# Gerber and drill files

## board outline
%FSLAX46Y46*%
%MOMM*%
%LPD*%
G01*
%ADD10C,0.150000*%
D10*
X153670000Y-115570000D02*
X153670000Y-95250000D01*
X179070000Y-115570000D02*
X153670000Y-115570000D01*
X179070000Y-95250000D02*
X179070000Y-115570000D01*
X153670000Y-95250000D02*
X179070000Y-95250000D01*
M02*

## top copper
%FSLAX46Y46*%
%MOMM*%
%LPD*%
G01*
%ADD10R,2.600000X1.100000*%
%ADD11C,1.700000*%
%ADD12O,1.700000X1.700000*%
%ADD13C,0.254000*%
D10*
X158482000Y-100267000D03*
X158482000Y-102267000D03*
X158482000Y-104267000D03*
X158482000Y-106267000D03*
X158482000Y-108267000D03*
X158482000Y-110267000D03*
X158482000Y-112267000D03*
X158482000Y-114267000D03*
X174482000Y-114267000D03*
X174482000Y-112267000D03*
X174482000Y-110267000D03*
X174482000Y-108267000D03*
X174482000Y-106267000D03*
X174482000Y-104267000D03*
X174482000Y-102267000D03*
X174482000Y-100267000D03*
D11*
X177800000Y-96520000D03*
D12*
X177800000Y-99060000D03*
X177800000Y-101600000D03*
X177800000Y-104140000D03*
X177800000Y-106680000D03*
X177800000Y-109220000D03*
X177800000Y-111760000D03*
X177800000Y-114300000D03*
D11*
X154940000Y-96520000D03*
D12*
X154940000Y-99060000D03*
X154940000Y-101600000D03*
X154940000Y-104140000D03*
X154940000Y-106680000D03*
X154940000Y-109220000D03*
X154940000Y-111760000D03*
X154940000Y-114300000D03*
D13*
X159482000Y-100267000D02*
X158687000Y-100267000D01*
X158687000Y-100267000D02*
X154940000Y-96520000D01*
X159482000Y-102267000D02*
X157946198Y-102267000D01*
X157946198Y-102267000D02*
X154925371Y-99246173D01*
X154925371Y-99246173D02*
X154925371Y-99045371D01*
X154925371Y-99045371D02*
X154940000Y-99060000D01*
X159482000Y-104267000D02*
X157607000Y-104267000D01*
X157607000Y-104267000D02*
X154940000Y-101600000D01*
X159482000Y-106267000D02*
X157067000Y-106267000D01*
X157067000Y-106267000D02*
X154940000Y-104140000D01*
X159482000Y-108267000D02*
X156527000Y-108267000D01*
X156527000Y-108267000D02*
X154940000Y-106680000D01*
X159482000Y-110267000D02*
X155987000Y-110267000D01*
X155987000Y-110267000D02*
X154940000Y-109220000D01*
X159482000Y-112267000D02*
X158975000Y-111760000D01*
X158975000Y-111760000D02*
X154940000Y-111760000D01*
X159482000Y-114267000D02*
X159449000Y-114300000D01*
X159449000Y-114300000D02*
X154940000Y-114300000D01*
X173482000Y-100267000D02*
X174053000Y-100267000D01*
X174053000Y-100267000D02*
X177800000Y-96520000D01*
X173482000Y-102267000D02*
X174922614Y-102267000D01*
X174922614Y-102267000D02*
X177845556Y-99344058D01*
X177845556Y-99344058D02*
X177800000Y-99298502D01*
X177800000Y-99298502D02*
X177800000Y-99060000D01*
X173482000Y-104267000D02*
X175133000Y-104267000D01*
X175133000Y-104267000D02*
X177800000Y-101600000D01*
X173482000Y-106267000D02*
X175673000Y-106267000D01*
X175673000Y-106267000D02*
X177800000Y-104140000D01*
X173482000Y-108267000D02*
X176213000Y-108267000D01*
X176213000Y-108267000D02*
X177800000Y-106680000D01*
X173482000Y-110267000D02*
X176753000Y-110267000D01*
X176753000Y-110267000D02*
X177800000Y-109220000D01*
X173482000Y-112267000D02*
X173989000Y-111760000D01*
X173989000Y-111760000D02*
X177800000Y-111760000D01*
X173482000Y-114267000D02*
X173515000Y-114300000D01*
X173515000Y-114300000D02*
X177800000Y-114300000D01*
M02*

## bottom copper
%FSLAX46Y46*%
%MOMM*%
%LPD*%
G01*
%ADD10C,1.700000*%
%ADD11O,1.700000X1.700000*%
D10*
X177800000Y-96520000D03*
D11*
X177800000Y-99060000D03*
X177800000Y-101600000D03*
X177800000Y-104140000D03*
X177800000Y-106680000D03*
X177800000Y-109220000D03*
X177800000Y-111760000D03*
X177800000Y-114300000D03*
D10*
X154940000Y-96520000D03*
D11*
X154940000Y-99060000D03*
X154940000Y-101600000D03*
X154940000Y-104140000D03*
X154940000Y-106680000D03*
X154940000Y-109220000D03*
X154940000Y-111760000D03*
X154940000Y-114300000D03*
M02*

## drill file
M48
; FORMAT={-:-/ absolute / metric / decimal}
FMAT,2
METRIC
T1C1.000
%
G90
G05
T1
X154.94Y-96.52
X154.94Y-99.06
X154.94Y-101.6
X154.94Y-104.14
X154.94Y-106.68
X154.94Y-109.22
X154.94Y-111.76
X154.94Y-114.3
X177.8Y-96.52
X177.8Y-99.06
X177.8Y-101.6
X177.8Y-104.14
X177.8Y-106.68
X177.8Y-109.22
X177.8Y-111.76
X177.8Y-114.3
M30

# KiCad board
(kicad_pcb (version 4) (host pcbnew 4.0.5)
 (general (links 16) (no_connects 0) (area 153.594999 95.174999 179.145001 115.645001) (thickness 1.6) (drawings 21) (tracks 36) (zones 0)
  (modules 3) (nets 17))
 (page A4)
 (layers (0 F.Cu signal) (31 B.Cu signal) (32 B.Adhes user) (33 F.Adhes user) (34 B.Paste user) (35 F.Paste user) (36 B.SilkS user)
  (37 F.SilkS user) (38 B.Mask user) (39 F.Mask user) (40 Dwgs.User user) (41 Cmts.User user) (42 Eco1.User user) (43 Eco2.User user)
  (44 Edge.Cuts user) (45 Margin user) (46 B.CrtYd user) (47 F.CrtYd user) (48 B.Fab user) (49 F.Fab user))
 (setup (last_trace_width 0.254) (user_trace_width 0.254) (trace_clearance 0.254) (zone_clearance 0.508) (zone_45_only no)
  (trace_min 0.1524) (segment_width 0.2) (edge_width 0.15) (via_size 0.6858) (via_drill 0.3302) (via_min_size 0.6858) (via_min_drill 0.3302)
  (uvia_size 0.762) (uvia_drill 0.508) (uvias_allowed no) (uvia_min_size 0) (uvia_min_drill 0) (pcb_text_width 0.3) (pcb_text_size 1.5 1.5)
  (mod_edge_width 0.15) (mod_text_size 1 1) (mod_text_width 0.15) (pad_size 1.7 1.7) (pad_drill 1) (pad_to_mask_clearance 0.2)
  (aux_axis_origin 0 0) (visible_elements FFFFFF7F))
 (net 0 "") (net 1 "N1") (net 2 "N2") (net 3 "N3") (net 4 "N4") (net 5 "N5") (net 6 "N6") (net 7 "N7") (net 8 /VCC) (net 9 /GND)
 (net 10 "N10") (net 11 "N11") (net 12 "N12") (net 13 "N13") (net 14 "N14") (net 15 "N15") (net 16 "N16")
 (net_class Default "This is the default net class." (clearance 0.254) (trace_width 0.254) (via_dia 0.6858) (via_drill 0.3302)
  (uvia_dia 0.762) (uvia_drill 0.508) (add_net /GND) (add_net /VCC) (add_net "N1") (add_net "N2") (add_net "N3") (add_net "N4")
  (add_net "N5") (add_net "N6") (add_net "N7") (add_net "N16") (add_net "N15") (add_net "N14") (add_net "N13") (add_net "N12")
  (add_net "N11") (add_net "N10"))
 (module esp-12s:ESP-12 (layer F.Cu) (at 159.482 100.267)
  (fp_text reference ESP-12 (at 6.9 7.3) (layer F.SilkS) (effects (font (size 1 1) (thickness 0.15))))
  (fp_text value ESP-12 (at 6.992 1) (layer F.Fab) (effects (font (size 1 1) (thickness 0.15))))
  (pad 1 smd rect (at 0 0) (size 2.6 1.1) (drill (offset -1 0)) (layers F.Cu F.Paste F.Mask) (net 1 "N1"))
  (pad 2 smd rect (at 0 2) (size 2.6 1.1) (drill (offset -1 0)) (layers F.Cu F.Paste F.Mask) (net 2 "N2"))
  (pad 3 smd rect (at 0 4) (size 2.6 1.1) (drill (offset -1 0)) (layers F.Cu F.Paste F.Mask) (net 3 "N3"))
  (pad 4 smd rect (at 0 6) (size 2.6 1.1) (drill (offset -1 0)) (layers F.Cu F.Paste F.Mask) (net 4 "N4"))
  (pad 5 smd rect (at 0 8) (size 2.6 1.1) (drill (offset -1 0)) (layers F.Cu F.Paste F.Mask) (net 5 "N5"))
  (pad 6 smd rect (at 0 10) (size 2.6 1.1) (drill (offset -1 0)) (layers F.Cu F.Paste F.Mask) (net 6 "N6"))
  (pad 7 smd rect (at 0 12) (size 2.6 1.1) (drill (offset -1 0)) (layers F.Cu F.Paste F.Mask) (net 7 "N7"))
  (pad 8 smd rect (at 0 14) (size 2.6 1.1) (drill (offset -1 0)) (layers F.Cu F.Paste F.Mask) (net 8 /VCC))
  (pad 9 smd rect (at 14 14) (size 2.6 1.1) (drill (offset 1 0)) (layers F.Cu F.Paste F.Mask) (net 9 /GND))
  (pad 10 smd rect (at 14 12) (size 2.6 1.1) (drill (offset 1 0)) (layers F.Cu F.Paste F.Mask) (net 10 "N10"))
  (pad 11 smd rect (at 14 10) (size 2.6 1.1) (drill (offset 1 0)) (layers F.Cu F.Paste F.Mask) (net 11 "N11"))
  (pad 12 smd rect (at 14 8) (size 2.6 1.1) (drill (offset 1 0)) (layers F.Cu F.Paste F.Mask) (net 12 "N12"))
  (pad 13 smd rect (at 14 6) (size 2.6 1.1) (drill (offset 1 0)) (layers F.Cu F.Paste F.Mask) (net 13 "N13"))
  (pad 14 smd rect (at 14 4) (size 2.6 1.1) (drill (offset 1 0)) (layers F.Cu F.Paste F.Mask) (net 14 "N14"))
  (pad 15 smd rect (at 14 2) (size 2.6 1.1) (drill (offset 1 0)) (layers F.Cu F.Paste F.Mask) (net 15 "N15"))
  (pad 16 smd rect (at 14 0) (size 2.6 1.1) (drill (offset 1 0)) (layers F.Cu F.Paste F.Mask) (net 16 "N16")))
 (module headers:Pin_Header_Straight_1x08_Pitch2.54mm (layer F.Cu) (at 177.8 96.52)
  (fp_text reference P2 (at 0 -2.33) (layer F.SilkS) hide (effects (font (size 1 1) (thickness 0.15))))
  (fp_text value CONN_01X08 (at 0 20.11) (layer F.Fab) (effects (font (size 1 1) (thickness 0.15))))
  (pad 1 thru_hole circle (at 0 0) (size 1.7 1.7) (drill 1) (layers *.Cu *.Mask) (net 16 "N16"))
  (pad 2 thru_hole oval (at 0 2.54) (size 1.7 1.7) (drill 1) (layers *.Cu *.Mask) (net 15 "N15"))
  (pad 3 thru_hole oval (at 0 5.08) (size 1.7 1.7) (drill 1) (layers *.Cu *.Mask) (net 14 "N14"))
  (pad 4 thru_hole oval (at 0 7.62) (size 1.7 1.7) (drill 1) (layers *.Cu *.Mask) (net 13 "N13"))
  (pad 5 thru_hole oval (at 0 10.16) (size 1.7 1.7) (drill 1) (layers *.Cu *.Mask) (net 12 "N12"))
  (pad 6 thru_hole oval (at 0 12.7) (size 1.7 1.7) (drill 1) (layers *.Cu *.Mask) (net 11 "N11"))
  (pad 7 thru_hole oval (at 0 15.24) (size 1.7 1.7) (drill 1) (layers *.Cu *.Mask) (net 10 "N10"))
  (pad 8 thru_hole oval (at 0 17.78) (size 1.7 1.7) (drill 1) (layers *.Cu *.Mask) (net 9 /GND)))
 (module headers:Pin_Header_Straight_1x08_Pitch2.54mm (layer F.Cu) (at 154.94 96.52)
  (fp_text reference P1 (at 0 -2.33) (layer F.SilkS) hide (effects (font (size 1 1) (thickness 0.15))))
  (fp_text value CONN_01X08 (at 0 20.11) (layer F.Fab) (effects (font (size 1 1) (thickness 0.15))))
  (pad 1 thru_hole circle (at 0 0) (size 1.7 1.7) (drill 1) (layers *.Cu *.Mask) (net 1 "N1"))
  (pad 2 thru_hole oval (at 0 2.54) (size 1.7 1.7) (drill 1) (layers *.Cu *.Mask) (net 2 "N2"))
  (pad 3 thru_hole oval (at 0 5.08) (size 1.7 1.7) (drill 1) (layers *.Cu *.Mask) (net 3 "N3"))
  (pad 4 thru_hole oval (at 0 7.62) (size 1.7 1.7) (drill 1) (layers *.Cu *.Mask) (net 4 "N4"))
  (pad 5 thru_hole oval (at 0 10.16) (size 1.7 1.7) (drill 1) (layers *.Cu *.Mask) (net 5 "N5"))
  (pad 6 thru_hole oval (at 0 12.7) (size 1.7 1.7) (drill 1) (layers *.Cu *.Mask) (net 6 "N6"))
  (pad 7 thru_hole oval (at 0 15.24) (size 1.7 1.7) (drill 1) (layers *.Cu *.Mask) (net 7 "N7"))
  (pad 8 thru_hole oval (at 0 17.78) (size 1.7 1.7) (drill 1) (layers *.Cu *.Mask) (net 8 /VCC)))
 (gr_line (start 153.67 115.57) (end 153.67 95.25) (layer Edge.Cuts) (width 0.15))
 (gr_line (start 179.07 115.57) (end 153.67 115.57) (layer Edge.Cuts) (width 0.15))
 (gr_line (start 179.07 95.25) (end 179.07 115.57) (layer Edge.Cuts) (width 0.15))
 (gr_line (start 153.67 95.25) (end 179.07 95.25) (layer Edge.Cuts) (width 0.15))
 (segment (start 159.482 100.267) (end 158.687 100.267) (width 0.254) (layer F.Cu) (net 1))
 (segment (start 158.687 100.267) (end 154.94 96.52) (width 0.254) (layer F.Cu) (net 1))
 (segment (start 159.482 102.267) (end 157.946198 102.267) (width 0.254) (layer F.Cu) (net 2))
 (segment (start 157.946198 102.267) (end 154.925371 99.246173) (width 0.254) (layer F.Cu) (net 2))
 (segment (start 154.925371 99.246173) (end 154.925371 99.045371) (width 0.254) (layer F.Cu) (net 2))
 (segment (start 154.925371 99.045371) (end 154.94 99.06) (width 0.254) (layer F.Cu) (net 2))
 (segment (start 159.482 104.267) (end 157.607 104.267) (width 0.254) (layer F.Cu) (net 3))
 (segment (start 157.607 104.267) (end 154.94 101.6) (width 0.254) (layer F.Cu) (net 3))
 (segment (start 159.482 106.267) (end 157.067 106.267) (width 0.254) (layer F.Cu) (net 4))
 (segment (start 157.067 106.267) (end 154.94 104.14) (width 0.254) (layer F.Cu) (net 4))
 (segment (start 159.482 108.267) (end 156.527 108.267) (width 0.254) (layer F.Cu) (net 5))
 (segment (start 156.527 108.267) (end 154.94 106.68) (width 0.254) (layer F.Cu) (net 5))
 (segment (start 159.482 110.267) (end 155.987 110.267) (width 0.254) (layer F.Cu) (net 6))
 (segment (start 155.987 110.267) (end 154.94 109.22) (width 0.254) (layer F.Cu) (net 6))
 (segment (start 159.482 112.267) (end 158.975 111.76) (width 0.254) (layer F.Cu) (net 7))
 (segment (start 158.975 111.76) (end 154.94 111.76) (width 0.254) (layer F.Cu) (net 7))
 (segment (start 159.482 114.267) (end 159.449 114.3) (width 0.254) (layer F.Cu) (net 8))
 (segment (start 159.449 114.3) (end 154.94 114.3) (width 0.254) (layer F.Cu) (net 8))
 (segment (start 173.482 100.267) (end 174.053 100.267) (width 0.254) (layer F.Cu) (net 16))
 (segment (start 174.053 100.267) (end 177.8 96.52) (width 0.254) (layer F.Cu) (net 16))
 (segment (start 173.482 102.267) (end 174.922614 102.267) (width 0.254) (layer F.Cu) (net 15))
 (segment (start 174.922614 102.267) (end 177.845556 99.344058) (width 0.254) (layer F.Cu) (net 15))
 (segment (start 177.845556 99.344058) (end 177.8 99.298502) (width 0.254) (layer F.Cu) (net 15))
 (segment (start 177.8 99.298502) (end 177.8 99.06) (width 0.254) (layer F.Cu) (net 15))
 (segment (start 173.482 104.267) (end 175.133 104.267) (width 0.254) (layer F.Cu) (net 14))
 (segment (start 175.133 104.267) (end 177.8 101.6) (width 0.254) (layer F.Cu) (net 14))
 (segment (start 173.482 106.267) (end 175.673 106.267) (width 0.254) (layer F.Cu) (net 13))
 (segment (start 175.673 106.267) (end 177.8 104.14) (width 0.254) (layer F.Cu) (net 13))
 (segment (start 173.482 108.267) (end 176.213 108.267) (width 0.254) (layer F.Cu) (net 12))
 (segment (start 176.213 108.267) (end 177.8 106.68) (width 0.254) (layer F.Cu) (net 12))
 (segment (start 173.482 110.267) (end 176.753 110.267) (width 0.254) (layer F.Cu) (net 11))
 (segment (start 176.753 110.267) (end 177.8 109.22) (width 0.254) (layer F.Cu) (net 11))
 (segment (start 173.482 112.267) (end 173.989 111.76) (width 0.254) (layer F.Cu) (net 10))
 (segment (start 173.989 111.76) (end 177.8 111.76) (width 0.254) (layer F.Cu) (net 10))
 (segment (start 173.482 114.267) (end 173.515 114.3) (width 0.254) (layer F.Cu) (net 9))
 (segment (start 173.515 114.3) (end 177.8 114.3) (width 0.254) (layer F.Cu) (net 9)))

